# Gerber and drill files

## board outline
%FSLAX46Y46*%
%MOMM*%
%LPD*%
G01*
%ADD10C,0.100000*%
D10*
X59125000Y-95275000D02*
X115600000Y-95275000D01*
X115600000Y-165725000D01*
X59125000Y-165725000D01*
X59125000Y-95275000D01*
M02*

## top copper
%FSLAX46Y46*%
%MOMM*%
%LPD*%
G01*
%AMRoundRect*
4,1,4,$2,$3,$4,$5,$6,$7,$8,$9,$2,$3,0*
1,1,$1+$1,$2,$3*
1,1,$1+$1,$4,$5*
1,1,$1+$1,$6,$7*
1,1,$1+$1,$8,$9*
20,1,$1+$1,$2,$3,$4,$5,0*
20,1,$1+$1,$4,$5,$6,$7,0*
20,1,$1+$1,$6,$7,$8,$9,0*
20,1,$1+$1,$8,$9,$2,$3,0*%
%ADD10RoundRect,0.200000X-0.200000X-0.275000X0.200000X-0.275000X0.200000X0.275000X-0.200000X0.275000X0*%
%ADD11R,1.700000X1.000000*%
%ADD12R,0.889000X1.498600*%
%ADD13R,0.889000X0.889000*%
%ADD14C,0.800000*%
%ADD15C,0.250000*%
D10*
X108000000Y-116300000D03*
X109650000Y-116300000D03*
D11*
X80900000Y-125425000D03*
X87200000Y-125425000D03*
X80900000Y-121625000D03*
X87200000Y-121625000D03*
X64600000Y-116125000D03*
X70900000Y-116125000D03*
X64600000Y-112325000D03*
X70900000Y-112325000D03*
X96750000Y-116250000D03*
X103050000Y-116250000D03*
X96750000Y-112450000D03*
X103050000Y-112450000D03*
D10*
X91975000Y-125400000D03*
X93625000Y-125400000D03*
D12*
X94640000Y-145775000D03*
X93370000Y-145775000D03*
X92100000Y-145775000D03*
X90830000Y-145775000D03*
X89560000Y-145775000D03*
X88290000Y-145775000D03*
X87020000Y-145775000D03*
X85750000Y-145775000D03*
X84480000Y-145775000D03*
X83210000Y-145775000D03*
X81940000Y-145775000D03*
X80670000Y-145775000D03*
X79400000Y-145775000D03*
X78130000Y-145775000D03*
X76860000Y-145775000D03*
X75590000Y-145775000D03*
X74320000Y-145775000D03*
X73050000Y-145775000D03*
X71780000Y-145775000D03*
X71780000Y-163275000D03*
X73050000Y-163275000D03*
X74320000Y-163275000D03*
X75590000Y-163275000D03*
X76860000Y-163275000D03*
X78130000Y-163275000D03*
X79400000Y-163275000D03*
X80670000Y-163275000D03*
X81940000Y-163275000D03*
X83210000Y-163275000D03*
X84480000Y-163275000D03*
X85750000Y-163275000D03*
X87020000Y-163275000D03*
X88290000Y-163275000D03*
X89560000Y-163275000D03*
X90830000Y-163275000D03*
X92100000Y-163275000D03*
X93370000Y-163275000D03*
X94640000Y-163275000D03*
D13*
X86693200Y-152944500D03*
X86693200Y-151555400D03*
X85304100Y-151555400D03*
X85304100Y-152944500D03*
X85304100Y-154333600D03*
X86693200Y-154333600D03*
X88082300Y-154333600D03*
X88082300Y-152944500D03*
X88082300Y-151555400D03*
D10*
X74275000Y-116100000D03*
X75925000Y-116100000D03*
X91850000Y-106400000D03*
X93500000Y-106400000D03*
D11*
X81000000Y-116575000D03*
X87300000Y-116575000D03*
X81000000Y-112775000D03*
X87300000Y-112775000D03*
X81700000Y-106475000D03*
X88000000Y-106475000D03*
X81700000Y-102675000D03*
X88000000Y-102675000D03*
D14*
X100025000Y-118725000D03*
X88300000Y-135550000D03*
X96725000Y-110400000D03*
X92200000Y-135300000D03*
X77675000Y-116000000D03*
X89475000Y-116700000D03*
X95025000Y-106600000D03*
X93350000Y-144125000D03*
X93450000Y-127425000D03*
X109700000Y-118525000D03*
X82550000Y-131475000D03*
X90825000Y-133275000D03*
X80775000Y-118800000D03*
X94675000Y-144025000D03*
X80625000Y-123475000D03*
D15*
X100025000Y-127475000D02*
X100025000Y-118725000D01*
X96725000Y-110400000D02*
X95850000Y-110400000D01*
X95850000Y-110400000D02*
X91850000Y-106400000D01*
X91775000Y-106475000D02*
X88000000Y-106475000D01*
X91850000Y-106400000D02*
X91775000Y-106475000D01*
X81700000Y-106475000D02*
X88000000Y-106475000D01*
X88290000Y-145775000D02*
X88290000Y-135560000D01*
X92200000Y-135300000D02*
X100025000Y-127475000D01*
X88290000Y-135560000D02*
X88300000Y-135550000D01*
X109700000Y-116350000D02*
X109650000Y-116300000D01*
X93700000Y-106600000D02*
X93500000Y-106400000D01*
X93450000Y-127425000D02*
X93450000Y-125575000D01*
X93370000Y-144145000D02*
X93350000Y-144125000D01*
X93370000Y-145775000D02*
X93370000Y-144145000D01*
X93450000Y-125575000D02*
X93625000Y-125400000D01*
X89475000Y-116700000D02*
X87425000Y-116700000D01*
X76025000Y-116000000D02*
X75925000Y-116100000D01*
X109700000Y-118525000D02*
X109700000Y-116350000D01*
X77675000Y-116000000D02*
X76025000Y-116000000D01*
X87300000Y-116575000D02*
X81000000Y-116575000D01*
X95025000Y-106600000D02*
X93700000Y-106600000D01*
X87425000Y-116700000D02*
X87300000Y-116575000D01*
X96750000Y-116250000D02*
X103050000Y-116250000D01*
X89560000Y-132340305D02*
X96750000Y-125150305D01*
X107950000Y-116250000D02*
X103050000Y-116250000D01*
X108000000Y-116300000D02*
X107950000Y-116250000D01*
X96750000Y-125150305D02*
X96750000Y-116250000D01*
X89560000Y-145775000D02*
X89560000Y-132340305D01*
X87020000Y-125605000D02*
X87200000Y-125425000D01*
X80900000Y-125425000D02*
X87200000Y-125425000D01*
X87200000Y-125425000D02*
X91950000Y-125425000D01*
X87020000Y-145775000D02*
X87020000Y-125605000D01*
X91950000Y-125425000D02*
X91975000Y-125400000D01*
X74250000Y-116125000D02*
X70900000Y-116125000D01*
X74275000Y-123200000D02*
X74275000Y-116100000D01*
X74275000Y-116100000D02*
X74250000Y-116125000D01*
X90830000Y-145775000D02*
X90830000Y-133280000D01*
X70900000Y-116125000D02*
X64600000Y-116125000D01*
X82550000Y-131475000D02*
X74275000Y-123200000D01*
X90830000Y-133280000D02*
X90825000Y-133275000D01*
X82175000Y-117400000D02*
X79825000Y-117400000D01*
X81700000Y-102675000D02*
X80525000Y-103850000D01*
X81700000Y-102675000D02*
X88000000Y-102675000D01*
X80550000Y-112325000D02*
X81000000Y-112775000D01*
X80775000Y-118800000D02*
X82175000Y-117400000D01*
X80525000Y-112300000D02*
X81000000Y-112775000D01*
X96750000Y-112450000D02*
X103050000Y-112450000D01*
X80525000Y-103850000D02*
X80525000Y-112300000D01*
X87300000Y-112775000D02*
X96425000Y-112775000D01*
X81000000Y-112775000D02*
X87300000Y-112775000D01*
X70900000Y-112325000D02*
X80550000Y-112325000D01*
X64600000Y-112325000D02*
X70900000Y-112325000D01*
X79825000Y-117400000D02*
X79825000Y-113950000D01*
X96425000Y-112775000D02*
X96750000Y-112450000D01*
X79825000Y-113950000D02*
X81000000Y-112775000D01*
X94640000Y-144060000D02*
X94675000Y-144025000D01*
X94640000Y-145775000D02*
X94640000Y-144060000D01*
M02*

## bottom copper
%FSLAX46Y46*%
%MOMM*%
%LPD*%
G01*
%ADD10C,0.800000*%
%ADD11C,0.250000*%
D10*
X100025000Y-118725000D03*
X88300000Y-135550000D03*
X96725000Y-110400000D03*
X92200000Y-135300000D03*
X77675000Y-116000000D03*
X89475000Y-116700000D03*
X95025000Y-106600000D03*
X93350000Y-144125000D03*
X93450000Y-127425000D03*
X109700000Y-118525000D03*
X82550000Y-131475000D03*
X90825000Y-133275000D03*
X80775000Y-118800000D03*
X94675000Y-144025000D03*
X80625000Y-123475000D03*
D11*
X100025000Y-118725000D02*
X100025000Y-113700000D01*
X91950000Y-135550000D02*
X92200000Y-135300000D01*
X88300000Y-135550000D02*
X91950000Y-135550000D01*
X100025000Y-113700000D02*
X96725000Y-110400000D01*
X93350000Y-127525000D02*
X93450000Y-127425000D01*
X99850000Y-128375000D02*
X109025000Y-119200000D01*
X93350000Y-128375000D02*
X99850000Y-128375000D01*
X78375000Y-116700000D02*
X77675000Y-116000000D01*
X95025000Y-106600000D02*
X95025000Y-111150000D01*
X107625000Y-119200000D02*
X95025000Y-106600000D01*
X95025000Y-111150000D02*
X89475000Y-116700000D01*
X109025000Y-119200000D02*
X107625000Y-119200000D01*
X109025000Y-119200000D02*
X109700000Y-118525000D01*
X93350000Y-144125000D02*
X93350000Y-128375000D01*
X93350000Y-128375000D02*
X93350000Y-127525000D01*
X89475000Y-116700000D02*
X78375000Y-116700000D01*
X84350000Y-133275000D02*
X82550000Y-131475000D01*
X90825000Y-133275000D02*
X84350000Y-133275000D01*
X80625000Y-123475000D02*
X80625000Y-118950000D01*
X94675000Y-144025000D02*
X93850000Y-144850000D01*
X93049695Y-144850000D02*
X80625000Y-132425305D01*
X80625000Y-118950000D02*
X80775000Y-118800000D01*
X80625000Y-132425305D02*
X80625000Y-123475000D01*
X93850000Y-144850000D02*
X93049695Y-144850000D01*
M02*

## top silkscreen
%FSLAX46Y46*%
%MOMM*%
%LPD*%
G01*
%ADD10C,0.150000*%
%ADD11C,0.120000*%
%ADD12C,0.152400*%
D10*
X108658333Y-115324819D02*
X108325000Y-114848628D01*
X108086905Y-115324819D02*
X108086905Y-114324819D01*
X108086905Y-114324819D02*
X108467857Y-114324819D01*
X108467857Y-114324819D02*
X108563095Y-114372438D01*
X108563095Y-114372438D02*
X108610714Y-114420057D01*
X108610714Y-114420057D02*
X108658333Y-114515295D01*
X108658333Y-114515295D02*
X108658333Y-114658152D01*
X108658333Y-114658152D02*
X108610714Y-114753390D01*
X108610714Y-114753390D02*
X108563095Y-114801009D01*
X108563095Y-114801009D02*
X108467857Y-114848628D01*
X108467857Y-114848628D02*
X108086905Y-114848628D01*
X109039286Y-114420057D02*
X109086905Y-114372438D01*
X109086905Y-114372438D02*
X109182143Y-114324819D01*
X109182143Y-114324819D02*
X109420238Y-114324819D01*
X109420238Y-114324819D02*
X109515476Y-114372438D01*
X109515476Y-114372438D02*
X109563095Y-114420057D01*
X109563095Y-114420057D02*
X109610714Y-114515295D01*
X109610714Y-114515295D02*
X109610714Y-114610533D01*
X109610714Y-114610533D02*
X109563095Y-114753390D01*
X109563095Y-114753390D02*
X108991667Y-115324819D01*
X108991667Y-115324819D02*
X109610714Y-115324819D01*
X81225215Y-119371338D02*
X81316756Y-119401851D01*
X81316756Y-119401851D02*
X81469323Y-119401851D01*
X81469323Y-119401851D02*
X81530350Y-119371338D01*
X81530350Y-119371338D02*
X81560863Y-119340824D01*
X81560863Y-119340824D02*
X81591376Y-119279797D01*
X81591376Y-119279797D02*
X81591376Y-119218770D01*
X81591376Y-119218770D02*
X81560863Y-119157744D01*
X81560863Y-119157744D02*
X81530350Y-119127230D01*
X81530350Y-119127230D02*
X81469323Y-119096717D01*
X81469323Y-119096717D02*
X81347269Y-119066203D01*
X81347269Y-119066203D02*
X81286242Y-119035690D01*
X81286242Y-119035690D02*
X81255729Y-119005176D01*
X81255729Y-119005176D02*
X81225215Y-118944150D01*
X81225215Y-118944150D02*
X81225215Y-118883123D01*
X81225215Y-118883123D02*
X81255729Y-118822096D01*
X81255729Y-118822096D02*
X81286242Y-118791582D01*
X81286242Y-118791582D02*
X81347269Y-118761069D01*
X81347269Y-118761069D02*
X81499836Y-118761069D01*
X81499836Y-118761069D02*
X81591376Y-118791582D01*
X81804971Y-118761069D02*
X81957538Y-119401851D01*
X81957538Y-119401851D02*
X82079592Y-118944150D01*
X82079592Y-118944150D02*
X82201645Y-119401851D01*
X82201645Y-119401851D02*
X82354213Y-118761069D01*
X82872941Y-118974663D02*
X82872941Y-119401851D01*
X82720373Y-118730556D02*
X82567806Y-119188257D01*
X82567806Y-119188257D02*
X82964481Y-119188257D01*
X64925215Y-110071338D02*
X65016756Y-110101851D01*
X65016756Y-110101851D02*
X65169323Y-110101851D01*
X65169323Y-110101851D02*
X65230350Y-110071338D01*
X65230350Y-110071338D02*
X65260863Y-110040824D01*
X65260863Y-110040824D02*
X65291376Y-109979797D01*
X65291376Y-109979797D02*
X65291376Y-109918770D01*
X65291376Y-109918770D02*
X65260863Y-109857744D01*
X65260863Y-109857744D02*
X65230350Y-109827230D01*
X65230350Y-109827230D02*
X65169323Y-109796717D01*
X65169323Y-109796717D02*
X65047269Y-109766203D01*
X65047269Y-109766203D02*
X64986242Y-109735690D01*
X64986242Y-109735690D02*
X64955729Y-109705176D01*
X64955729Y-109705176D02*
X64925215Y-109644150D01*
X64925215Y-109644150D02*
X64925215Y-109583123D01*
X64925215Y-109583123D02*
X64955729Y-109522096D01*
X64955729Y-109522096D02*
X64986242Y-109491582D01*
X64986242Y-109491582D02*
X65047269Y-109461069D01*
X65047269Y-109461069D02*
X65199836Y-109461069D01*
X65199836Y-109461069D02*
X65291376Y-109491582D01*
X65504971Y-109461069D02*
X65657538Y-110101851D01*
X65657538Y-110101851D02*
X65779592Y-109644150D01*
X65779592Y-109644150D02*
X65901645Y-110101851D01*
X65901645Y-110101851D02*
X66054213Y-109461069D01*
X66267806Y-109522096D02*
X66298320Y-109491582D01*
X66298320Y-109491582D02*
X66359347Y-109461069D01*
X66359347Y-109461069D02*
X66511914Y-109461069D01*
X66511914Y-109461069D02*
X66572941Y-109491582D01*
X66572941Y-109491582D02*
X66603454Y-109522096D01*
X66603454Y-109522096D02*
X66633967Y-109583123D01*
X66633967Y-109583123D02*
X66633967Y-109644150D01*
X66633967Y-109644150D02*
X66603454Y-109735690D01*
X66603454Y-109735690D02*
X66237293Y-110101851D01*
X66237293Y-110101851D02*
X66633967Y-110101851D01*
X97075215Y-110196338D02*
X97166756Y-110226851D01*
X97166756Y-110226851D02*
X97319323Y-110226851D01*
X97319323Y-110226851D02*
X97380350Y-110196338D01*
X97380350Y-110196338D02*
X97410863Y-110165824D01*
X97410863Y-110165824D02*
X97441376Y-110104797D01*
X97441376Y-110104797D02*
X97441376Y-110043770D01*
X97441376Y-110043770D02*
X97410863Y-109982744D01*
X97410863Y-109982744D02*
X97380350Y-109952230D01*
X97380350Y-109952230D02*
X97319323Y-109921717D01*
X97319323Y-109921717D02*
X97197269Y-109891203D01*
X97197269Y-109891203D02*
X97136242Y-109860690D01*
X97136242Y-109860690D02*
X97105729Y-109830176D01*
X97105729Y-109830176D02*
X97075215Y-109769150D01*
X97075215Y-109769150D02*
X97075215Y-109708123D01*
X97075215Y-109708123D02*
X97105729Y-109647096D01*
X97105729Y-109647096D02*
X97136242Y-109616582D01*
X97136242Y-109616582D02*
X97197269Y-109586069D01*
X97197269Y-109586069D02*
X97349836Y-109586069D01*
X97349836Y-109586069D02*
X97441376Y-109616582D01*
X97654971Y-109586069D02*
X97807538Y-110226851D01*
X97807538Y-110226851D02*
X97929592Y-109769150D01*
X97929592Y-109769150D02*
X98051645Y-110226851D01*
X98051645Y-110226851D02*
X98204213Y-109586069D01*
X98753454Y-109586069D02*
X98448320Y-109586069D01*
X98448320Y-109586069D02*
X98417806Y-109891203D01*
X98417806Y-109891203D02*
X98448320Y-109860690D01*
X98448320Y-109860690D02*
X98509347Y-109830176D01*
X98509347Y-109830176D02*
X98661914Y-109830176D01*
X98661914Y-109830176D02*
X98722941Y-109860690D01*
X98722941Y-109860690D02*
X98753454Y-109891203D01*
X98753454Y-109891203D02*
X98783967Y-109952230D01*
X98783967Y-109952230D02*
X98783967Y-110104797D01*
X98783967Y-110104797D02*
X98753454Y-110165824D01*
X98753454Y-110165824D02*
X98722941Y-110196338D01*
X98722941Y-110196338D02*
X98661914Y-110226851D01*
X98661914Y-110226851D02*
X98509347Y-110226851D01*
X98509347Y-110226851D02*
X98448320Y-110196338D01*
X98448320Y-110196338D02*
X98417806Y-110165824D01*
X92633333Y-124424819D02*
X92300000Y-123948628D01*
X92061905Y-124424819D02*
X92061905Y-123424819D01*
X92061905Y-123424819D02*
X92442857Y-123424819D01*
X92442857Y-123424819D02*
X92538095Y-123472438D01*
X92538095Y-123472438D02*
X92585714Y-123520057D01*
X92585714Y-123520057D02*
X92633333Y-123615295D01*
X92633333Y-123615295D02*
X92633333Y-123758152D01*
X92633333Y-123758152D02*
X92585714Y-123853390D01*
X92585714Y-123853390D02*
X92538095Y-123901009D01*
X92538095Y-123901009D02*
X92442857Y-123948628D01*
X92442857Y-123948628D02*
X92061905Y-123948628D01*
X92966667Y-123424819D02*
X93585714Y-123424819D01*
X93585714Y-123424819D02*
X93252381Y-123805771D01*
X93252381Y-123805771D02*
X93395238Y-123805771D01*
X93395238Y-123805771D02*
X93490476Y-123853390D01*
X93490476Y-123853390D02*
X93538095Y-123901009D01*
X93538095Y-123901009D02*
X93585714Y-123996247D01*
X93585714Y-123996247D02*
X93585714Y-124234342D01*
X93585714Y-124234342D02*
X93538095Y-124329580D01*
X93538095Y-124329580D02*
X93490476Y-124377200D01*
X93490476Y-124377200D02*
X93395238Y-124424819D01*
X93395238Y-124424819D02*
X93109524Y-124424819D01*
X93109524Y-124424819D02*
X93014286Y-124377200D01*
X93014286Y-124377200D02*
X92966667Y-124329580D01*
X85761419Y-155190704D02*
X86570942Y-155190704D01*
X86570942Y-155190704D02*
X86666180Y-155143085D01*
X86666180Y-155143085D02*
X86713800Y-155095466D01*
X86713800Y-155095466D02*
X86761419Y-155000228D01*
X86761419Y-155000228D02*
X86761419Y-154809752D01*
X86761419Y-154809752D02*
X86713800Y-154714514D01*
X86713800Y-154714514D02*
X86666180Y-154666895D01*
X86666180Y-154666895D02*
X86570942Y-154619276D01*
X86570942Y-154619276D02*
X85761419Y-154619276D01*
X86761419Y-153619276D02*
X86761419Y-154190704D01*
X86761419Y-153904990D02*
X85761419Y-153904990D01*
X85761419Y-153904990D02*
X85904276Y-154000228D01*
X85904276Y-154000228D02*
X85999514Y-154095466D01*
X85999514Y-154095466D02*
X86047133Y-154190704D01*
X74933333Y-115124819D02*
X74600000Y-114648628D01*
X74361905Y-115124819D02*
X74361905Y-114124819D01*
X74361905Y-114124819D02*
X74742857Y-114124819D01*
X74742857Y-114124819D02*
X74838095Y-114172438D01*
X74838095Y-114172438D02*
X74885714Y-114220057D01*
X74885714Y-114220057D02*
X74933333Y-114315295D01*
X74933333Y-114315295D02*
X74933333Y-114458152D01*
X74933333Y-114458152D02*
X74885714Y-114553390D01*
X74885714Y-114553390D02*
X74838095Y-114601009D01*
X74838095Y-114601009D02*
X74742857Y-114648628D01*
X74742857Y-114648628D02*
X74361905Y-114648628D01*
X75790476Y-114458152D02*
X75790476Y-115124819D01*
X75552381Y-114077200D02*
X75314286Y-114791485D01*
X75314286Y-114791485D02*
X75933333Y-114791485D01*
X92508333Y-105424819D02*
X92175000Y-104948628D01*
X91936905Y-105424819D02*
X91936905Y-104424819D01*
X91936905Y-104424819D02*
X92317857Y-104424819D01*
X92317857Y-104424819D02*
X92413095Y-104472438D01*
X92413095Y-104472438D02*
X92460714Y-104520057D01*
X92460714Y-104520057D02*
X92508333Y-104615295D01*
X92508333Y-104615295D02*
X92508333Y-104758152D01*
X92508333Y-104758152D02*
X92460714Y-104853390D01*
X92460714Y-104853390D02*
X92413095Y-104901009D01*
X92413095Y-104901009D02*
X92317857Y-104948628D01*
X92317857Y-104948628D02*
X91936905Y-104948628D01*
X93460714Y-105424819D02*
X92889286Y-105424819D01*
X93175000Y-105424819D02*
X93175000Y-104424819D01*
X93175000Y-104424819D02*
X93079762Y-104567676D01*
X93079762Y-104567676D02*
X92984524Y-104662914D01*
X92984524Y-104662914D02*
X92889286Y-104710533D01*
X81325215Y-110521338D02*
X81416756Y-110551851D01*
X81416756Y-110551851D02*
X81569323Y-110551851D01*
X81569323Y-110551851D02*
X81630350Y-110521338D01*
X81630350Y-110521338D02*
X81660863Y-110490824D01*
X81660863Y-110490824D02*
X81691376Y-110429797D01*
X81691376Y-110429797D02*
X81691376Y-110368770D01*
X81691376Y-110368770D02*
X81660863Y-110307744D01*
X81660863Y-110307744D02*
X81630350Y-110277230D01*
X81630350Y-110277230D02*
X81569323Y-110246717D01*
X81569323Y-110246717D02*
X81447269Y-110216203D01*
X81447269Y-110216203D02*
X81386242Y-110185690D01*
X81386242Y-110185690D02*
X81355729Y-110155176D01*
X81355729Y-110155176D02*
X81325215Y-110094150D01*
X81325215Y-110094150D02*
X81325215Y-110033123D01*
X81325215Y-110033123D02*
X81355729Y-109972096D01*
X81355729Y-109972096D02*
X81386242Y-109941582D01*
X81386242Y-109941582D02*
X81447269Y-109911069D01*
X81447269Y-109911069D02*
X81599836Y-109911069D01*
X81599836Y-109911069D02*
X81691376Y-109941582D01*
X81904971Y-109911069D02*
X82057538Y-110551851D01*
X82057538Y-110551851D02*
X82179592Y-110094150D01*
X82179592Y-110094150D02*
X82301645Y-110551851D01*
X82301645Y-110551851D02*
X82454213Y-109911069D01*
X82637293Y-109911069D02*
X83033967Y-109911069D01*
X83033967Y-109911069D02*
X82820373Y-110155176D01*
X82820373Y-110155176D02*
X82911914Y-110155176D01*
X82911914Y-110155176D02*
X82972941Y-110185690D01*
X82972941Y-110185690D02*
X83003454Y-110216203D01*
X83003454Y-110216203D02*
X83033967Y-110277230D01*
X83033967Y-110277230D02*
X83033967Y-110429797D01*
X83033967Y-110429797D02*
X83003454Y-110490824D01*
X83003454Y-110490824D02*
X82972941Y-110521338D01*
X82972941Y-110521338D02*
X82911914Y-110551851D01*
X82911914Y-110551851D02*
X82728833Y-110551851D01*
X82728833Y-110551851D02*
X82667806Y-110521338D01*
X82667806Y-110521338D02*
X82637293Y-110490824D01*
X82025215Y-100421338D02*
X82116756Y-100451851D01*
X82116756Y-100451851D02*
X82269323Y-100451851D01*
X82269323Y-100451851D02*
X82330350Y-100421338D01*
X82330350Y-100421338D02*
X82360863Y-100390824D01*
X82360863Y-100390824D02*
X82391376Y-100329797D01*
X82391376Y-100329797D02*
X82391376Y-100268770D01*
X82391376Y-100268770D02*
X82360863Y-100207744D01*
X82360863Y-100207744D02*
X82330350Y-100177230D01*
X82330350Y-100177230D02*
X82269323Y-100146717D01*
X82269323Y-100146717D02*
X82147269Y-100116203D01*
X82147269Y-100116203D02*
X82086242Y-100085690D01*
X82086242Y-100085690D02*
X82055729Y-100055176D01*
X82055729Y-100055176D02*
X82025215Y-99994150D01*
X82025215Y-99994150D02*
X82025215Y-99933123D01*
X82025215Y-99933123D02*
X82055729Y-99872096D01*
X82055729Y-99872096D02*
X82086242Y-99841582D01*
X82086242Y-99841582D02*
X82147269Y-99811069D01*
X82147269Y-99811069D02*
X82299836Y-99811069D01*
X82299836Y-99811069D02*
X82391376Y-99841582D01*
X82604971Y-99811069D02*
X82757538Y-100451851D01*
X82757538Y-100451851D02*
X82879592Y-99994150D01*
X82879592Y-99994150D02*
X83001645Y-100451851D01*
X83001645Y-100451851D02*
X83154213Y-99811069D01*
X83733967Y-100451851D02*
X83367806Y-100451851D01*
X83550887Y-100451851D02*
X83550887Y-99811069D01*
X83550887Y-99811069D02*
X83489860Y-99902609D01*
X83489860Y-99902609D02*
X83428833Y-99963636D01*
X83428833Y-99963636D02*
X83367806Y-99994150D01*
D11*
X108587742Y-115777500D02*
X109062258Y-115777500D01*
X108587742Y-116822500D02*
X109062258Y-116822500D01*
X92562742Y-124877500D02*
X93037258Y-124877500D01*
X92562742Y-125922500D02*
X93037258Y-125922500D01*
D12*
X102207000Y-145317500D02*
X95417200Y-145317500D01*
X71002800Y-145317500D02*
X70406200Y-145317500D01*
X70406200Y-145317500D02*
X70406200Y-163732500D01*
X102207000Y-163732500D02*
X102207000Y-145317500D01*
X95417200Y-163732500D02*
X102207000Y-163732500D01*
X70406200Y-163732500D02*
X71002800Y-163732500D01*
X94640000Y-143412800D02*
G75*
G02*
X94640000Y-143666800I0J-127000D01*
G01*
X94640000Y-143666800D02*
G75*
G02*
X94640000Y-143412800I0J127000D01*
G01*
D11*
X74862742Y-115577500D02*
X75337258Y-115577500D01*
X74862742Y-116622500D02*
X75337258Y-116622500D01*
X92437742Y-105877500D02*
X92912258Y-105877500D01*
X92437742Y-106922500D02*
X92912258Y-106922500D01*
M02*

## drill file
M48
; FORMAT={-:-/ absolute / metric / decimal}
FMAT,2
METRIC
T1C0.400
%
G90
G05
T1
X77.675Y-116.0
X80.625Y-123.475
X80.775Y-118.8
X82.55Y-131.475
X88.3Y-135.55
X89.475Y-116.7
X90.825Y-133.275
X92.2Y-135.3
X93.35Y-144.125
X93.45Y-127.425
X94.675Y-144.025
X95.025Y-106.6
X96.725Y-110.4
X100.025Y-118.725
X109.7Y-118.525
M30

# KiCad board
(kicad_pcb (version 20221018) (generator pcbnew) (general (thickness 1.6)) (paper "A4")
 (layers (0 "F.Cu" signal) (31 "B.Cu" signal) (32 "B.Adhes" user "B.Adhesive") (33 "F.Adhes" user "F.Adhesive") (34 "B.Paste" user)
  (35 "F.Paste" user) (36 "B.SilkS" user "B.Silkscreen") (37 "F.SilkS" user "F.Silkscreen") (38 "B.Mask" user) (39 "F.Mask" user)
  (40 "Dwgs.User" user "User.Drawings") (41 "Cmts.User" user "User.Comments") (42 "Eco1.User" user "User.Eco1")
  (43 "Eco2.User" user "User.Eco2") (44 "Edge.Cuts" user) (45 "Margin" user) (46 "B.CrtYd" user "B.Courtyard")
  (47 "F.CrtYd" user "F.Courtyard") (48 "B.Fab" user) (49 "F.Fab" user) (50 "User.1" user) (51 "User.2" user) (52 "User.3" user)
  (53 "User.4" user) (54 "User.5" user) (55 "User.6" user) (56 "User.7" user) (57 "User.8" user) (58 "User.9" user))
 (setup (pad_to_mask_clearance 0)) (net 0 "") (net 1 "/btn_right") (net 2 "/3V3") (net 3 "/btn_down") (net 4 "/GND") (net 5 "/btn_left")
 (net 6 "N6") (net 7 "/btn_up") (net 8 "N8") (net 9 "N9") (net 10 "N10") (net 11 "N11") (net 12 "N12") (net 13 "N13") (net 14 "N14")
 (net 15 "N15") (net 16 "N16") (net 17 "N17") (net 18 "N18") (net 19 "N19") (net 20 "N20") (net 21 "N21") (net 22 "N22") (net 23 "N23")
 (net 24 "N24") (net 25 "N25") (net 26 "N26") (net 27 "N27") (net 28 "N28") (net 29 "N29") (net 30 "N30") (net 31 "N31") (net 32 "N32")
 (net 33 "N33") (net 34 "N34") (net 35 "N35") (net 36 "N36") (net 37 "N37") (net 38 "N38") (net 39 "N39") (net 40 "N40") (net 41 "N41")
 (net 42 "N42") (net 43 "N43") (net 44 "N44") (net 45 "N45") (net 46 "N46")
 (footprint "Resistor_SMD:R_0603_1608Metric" (layer "F.Cu") (at 108.825 116.3)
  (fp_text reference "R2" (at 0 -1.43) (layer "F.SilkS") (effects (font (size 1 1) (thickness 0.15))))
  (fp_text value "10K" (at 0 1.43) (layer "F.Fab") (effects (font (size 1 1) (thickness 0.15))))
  (fp_line (start -0.237258 -0.5225) (end 0.237258 -0.5225) (stroke (width 0.12) (type solid)) (layer "F.SilkS"))
  (fp_line (start -0.237258 0.5225) (end 0.237258 0.5225) (stroke (width 0.12) (type solid)) (layer "F.SilkS"))
  (pad "1" smd roundrect (at -0.825 0) (size 0.8 0.95) (layers "F.Cu" "F.Paste" "F.Mask") (roundrect_rratio 0.25) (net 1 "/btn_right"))
  (pad "2" smd roundrect (at 0.825 0) (size 0.8 0.95) (layers "F.Cu" "F.Paste" "F.Mask") (roundrect_rratio 0.25) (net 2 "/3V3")))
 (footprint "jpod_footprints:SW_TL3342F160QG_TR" (layer "F.Cu") (at 84.05 123.525)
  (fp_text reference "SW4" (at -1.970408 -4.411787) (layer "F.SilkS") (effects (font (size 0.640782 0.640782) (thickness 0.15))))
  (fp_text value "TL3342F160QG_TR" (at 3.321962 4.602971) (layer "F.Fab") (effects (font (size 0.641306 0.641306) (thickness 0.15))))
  (pad "1" smd rect (at -3.15 1.9) (size 1.7 1) (layers "F.Cu" "F.Paste" "F.Mask") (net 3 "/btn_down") (solder_mask_margin 0.102))
  (pad "2" smd rect (at 3.15 1.9) (size 1.7 1) (layers "F.Cu" "F.Paste" "F.Mask") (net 3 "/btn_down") (solder_mask_margin 0.102))
  (pad "3" smd rect (at -3.15 -1.9) (size 1.7 1) (layers "F.Cu" "F.Paste" "F.Mask") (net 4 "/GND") (solder_mask_margin 0.102))
  (pad "4" smd rect (at 3.15 -1.9) (size 1.7 1) (layers "F.Cu" "F.Paste" "F.Mask") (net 4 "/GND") (solder_mask_margin 0.102)))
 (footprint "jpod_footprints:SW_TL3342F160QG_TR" (layer "F.Cu") (at 67.75 114.225)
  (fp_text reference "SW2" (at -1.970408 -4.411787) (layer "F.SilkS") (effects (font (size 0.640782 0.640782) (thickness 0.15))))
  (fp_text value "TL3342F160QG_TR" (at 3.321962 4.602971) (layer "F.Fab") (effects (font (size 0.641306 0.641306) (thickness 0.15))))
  (pad "1" smd rect (at -3.15 1.9) (size 1.7 1) (layers "F.Cu" "F.Paste" "F.Mask") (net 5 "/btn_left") (solder_mask_margin 0.102))
  (pad "2" smd rect (at 3.15 1.9) (size 1.7 1) (layers "F.Cu" "F.Paste" "F.Mask") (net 5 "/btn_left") (solder_mask_margin 0.102))
  (pad "3" smd rect (at -3.15 -1.9) (size 1.7 1) (layers "F.Cu" "F.Paste" "F.Mask") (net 4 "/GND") (solder_mask_margin 0.102))
  (pad "4" smd rect (at 3.15 -1.9) (size 1.7 1) (layers "F.Cu" "F.Paste" "F.Mask") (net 4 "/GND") (solder_mask_margin 0.102)))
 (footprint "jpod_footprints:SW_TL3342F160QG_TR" (layer "F.Cu") (at 99.9 114.35)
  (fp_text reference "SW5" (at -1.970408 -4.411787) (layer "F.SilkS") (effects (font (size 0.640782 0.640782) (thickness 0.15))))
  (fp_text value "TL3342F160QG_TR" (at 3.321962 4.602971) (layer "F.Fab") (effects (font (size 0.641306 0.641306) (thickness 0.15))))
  (pad "1" smd rect (at -3.15 1.9) (size 1.7 1) (layers "F.Cu" "F.Paste" "F.Mask") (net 1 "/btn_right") (solder_mask_margin 0.102))
  (pad "2" smd rect (at 3.15 1.9) (size 1.7 1) (layers "F.Cu" "F.Paste" "F.Mask") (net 1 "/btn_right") (solder_mask_margin 0.102))
  (pad "3" smd rect (at -3.15 -1.9) (size 1.7 1) (layers "F.Cu" "F.Paste" "F.Mask") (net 4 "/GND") (solder_mask_margin 0.102))
  (pad "4" smd rect (at 3.15 -1.9) (size 1.7 1) (layers "F.Cu" "F.Paste" "F.Mask") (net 4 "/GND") (solder_mask_margin 0.102)))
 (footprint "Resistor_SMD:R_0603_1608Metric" (layer "F.Cu") (at 92.8 125.4)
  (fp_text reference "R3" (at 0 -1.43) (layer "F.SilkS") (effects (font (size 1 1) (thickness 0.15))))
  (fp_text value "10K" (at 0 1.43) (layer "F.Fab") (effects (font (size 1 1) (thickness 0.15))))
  (fp_line (start -0.237258 -0.5225) (end 0.237258 -0.5225) (stroke (width 0.12) (type solid)) (layer "F.SilkS"))
  (fp_line (start -0.237258 0.5225) (end 0.237258 0.5225) (stroke (width 0.12) (type solid)) (layer "F.SilkS"))
  (pad "1" smd roundrect (at -0.825 0) (size 0.8 0.95) (layers "F.Cu" "F.Paste" "F.Mask") (roundrect_rratio 0.25) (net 3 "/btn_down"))
  (pad "2" smd roundrect (at 0.825 0) (size 0.8 0.95) (layers "F.Cu" "F.Paste" "F.Mask") (roundrect_rratio 0.25) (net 2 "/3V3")))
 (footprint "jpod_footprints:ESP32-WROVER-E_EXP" (layer "F.Cu") (at 86.3066 154.525 -90)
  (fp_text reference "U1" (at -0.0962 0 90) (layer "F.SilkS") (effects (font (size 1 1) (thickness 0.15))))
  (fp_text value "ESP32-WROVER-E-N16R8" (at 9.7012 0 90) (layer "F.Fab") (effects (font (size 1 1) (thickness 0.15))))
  (fp_line (start -9.2075 -15.9004) (end -9.2075 -9.1106) (stroke (width 0.1524) (type solid)) (layer "F.SilkS"))
  (fp_line (start -9.2075 15.3038) (end -9.2075 15.9004) (stroke (width 0.1524) (type solid)) (layer "F.SilkS"))
  (fp_line (start -9.2075 15.9004) (end 9.2075 15.9004) (stroke (width 0.1524) (type solid)) (layer "F.SilkS"))
  (fp_line (start 9.2075 -15.9004) (end -9.2075 -15.9004) (stroke (width 0.1524) (type solid)) (layer "F.SilkS"))
  (fp_line (start 9.2075 -9.1106) (end 9.2075 -15.9004) (stroke (width 0.1524) (type solid)) (layer "F.SilkS"))
  (fp_line (start 9.2075 15.9004) (end 9.2075 15.3038) (stroke (width 0.1524) (type solid)) (layer "F.SilkS"))
  (fp_arc (start -11.1122 -8.3334) (mid -10.9852 -8.4604) (end -10.8582 -8.3334) (stroke (width 0.1524) (type solid)) (layer "F.SilkS"))
  (fp_arc (start -10.8582 -8.3334) (mid -10.9852 -8.2064) (end -11.1122 -8.3334) (stroke (width 0.1524) (type solid)) (layer "F.SilkS"))
  (pad "1" smd rect (at -8.75 -8.3334 270) (size 1.4986 0.889) (layers "F.Cu" "F.Paste" "F.Mask") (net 4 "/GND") (solder_mask_margin 0.102))
  (pad "2" smd rect (at -8.75 -7.0634 270) (size 1.4986 0.889) (layers "F.Cu" "F.Paste" "F.Mask") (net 2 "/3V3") (solder_mask_margin 0.102))
  (pad "3" smd rect (at -8.75 -5.7934 270) (size 1.4986 0.889) (layers "F.Cu" "F.Paste" "F.Mask") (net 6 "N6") (solder_mask_margin 0.102))
  (pad "4" smd rect (at -8.75 -4.5234 270) (size 1.4986 0.889) (layers "F.Cu" "F.Paste" "F.Mask") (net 5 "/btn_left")
   (solder_mask_margin 0.102))
  (pad "5" smd rect (at -8.75 -3.2534 270) (size 1.4986 0.889) (layers "F.Cu" "F.Paste" "F.Mask") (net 1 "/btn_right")
   (solder_mask_margin 0.102))
  (pad "6" smd rect (at -8.75 -1.9834 270) (size 1.4986 0.889) (layers "F.Cu" "F.Paste" "F.Mask") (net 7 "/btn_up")
   (solder_mask_margin 0.102))
  (pad "7" smd rect (at -8.75 -0.7134 270) (size 1.4986 0.889) (layers "F.Cu" "F.Paste" "F.Mask") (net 3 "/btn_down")
   (solder_mask_margin 0.102))
  (pad "8" smd rect (at -8.75 0.5566 270) (size 1.4986 0.889) (layers "F.Cu" "F.Paste" "F.Mask") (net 2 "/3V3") (solder_mask_margin 0.102))
  (pad "9" smd rect (at -8.75 1.8266 270) (size 1.4986 0.889) (layers "F.Cu" "F.Paste" "F.Mask") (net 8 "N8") (solder_mask_margin 0.102))
  (pad "10" smd rect (at -8.75 3.0966 270) (size 1.4986 0.889) (layers "F.Cu" "F.Paste" "F.Mask") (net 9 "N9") (solder_mask_margin 0.102))
  (pad "11" smd rect (at -8.75 4.3666 270) (size 1.4986 0.889) (layers "F.Cu" "F.Paste" "F.Mask") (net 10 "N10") (solder_mask_margin 0.102))
  (pad "12" smd rect (at -8.75 5.6366 270) (size 1.4986 0.889) (layers "F.Cu" "F.Paste" "F.Mask") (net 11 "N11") (solder_mask_margin 0.102))
  (pad "13" smd rect (at -8.75 6.9066 270) (size 1.4986 0.889) (layers "F.Cu" "F.Paste" "F.Mask") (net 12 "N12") (solder_mask_margin 0.102))
  (pad "14" smd rect (at -8.75 8.1766 270) (size 1.4986 0.889) (layers "F.Cu" "F.Paste" "F.Mask") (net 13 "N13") (solder_mask_margin 0.102))
  (pad "15" smd rect (at -8.75 9.4466 270) (size 1.4986 0.889) (layers "F.Cu" "F.Paste" "F.Mask") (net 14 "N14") (solder_mask_margin 0.102))
  (pad "16" smd rect (at -8.75 10.7166 270) (size 1.4986 0.889) (layers "F.Cu" "F.Paste" "F.Mask") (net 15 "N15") (solder_mask_margin 0.102))
  (pad "17" smd rect (at -8.75 11.9866 270) (size 1.4986 0.889) (layers "F.Cu" "F.Paste" "F.Mask") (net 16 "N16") (solder_mask_margin 0.102))
  (pad "18" smd rect (at -8.75 13.2566 270) (size 1.4986 0.889) (layers "F.Cu" "F.Paste" "F.Mask") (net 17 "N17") (solder_mask_margin 0.102))
  (pad "19" smd rect (at -8.75 14.5266 270) (size 1.4986 0.889) (layers "F.Cu" "F.Paste" "F.Mask") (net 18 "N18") (solder_mask_margin 0.102))
  (pad "20" smd rect (at 8.75 14.5266 270) (size 1.4986 0.889) (layers "F.Cu" "F.Paste" "F.Mask") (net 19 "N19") (solder_mask_margin 0.102))
  (pad "21" smd rect (at 8.75 13.2566 270) (size 1.4986 0.889) (layers "F.Cu" "F.Paste" "F.Mask") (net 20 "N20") (solder_mask_margin 0.102))
  (pad "22" smd rect (at 8.75 11.9866 270) (size 1.4986 0.889) (layers "F.Cu" "F.Paste" "F.Mask") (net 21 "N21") (solder_mask_margin 0.102))
  (pad "23" smd rect (at 8.75 10.7166 270) (size 1.4986 0.889) (layers "F.Cu" "F.Paste" "F.Mask") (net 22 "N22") (solder_mask_margin 0.102))
  (pad "24" smd rect (at 8.75 9.4466 270) (size 1.4986 0.889) (layers "F.Cu" "F.Paste" "F.Mask") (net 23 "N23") (solder_mask_margin 0.102))
  (pad "25" smd rect (at 8.75 8.1766 270) (size 1.4986 0.889) (layers "F.Cu" "F.Paste" "F.Mask") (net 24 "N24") (solder_mask_margin 0.102))
  (pad "26" smd rect (at 8.75 6.9066 270) (size 1.4986 0.889) (layers "F.Cu" "F.Paste" "F.Mask") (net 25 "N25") (solder_mask_margin 0.102))
  (pad "27" smd rect (at 8.75 5.6366 270) (size 1.4986 0.889) (layers "F.Cu" "F.Paste" "F.Mask") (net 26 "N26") (solder_mask_margin 0.102))
  (pad "28" smd rect (at 8.75 4.3666 270) (size 1.4986 0.889) (layers "F.Cu" "F.Paste" "F.Mask") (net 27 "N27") (solder_mask_margin 0.102))
  (pad "29" smd rect (at 8.75 3.0966 270) (size 1.4986 0.889) (layers "F.Cu" "F.Paste" "F.Mask") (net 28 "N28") (solder_mask_margin 0.102))
  (pad "30" smd rect (at 8.75 1.8266 270) (size 1.4986 0.889) (layers "F.Cu" "F.Paste" "F.Mask") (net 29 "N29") (solder_mask_margin 0.102))
  (pad "31" smd rect (at 8.75 0.5566 270) (size 1.4986 0.889) (layers "F.Cu" "F.Paste" "F.Mask") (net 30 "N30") (solder_mask_margin 0.102))
  (pad "32" smd rect (at 8.75 -0.7134 270) (size 1.4986 0.889) (layers "F.Cu" "F.Paste" "F.Mask") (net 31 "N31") (solder_mask_margin 0.102))
  (pad "33" smd rect (at 8.75 -1.9834 270) (size 1.4986 0.889) (layers "F.Cu" "F.Paste" "F.Mask") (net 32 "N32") (solder_mask_margin 0.102))
  (pad "34" smd rect (at 8.75 -3.2534 270) (size 1.4986 0.889) (layers "F.Cu" "F.Paste" "F.Mask") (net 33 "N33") (solder_mask_margin 0.102))
  (pad "35" smd rect (at 8.75 -4.5234 270) (size 1.4986 0.889) (layers "F.Cu" "F.Paste" "F.Mask") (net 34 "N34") (solder_mask_margin 0.102))
  (pad "36" smd rect (at 8.75 -5.7934 270) (size 1.4986 0.889) (layers "F.Cu" "F.Paste" "F.Mask") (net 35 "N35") (solder_mask_margin 0.102))
  (pad "37" smd rect (at 8.75 -7.0634 270) (size 1.4986 0.889) (layers "F.Cu" "F.Paste" "F.Mask") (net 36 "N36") (solder_mask_margin 0.102))
  (pad "38" smd rect (at 8.75 -8.3334 270) (size 1.4986 0.889) (layers "F.Cu" "F.Paste" "F.Mask") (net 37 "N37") (solder_mask_margin 0.102))
  (pad "39" smd rect (at -1.5805 -0.3866 270) (size 0.889 0.889) (layers "F.Cu" "F.Paste" "F.Mask") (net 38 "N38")
   (solder_mask_margin 0.102))
  (pad "40" smd rect (at -2.9696 -0.3866 270) (size 0.889 0.889) (layers "F.Cu" "F.Paste" "F.Mask") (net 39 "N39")
   (solder_mask_margin 0.102))
  (pad "41" smd rect (at -2.9696 1.0025 270) (size 0.889 0.889) (layers "F.Cu" "F.Paste" "F.Mask") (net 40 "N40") (solder_mask_margin 0.102))
  (pad "42" smd rect (at -1.5805 1.0025 270) (size 0.889 0.889) (layers "F.Cu" "F.Paste" "F.Mask") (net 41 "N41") (solder_mask_margin 0.102))
  (pad "43" smd rect (at -0.1914 1.0025 270) (size 0.889 0.889) (layers "F.Cu" "F.Paste" "F.Mask") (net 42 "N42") (solder_mask_margin 0.102))
  (pad "44" smd rect (at -0.1914 -0.3866 270) (size 0.889 0.889) (layers "F.Cu" "F.Paste" "F.Mask") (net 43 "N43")
   (solder_mask_margin 0.102))
  (pad "45" smd rect (at -0.1914 -1.7757 270) (size 0.889 0.889) (layers "F.Cu" "F.Paste" "F.Mask") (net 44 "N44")
   (solder_mask_margin 0.102))
  (pad "46" smd rect (at -1.5805 -1.7757 270) (size 0.889 0.889) (layers "F.Cu" "F.Paste" "F.Mask") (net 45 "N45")
   (solder_mask_margin 0.102))
  (pad "47" smd rect (at -2.9696 -1.7757 270) (size 0.889 0.889) (layers "F.Cu" "F.Paste" "F.Mask") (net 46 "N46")
   (solder_mask_margin 0.102)))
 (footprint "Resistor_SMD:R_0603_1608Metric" (layer "F.Cu") (at 75.1 116.1)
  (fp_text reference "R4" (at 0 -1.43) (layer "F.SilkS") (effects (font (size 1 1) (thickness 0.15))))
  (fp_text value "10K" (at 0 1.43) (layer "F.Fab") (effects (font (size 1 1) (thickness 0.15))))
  (fp_line (start -0.237258 -0.5225) (end 0.237258 -0.5225) (stroke (width 0.12) (type solid)) (layer "F.SilkS"))
  (fp_line (start -0.237258 0.5225) (end 0.237258 0.5225) (stroke (width 0.12) (type solid)) (layer "F.SilkS"))
  (pad "1" smd roundrect (at -0.825 0) (size 0.8 0.95) (layers "F.Cu" "F.Paste" "F.Mask") (roundrect_rratio 0.25) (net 5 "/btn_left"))
  (pad "2" smd roundrect (at 0.825 0) (size 0.8 0.95) (layers "F.Cu" "F.Paste" "F.Mask") (roundrect_rratio 0.25) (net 2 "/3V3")))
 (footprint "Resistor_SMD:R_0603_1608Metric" (layer "F.Cu") (at 92.675 106.4)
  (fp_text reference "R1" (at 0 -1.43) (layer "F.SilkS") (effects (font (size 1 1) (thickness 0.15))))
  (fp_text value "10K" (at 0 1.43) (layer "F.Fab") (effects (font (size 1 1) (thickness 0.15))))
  (fp_line (start -0.237258 -0.5225) (end 0.237258 -0.5225) (stroke (width 0.12) (type solid)) (layer "F.SilkS"))
  (fp_line (start -0.237258 0.5225) (end 0.237258 0.5225) (stroke (width 0.12) (type solid)) (layer "F.SilkS"))
  (pad "1" smd roundrect (at -0.825 0) (size 0.8 0.95) (layers "F.Cu" "F.Paste" "F.Mask") (roundrect_rratio 0.25) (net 7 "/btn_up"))
  (pad "2" smd roundrect (at 0.825 0) (size 0.8 0.95) (layers "F.Cu" "F.Paste" "F.Mask") (roundrect_rratio 0.25) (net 2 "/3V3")))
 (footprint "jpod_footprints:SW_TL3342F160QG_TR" (layer "F.Cu") (at 84.15 114.675)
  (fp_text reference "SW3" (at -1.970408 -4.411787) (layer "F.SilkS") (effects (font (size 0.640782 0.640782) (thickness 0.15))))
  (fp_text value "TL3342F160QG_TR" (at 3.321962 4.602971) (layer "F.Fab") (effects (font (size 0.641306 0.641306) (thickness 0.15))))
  (pad "1" smd rect (at -3.15 1.9) (size 1.7 1) (layers "F.Cu" "F.Paste" "F.Mask") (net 2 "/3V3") (solder_mask_margin 0.102))
  (pad "2" smd rect (at 3.15 1.9) (size 1.7 1) (layers "F.Cu" "F.Paste" "F.Mask") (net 2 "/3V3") (solder_mask_margin 0.102))
  (pad "3" smd rect (at -3.15 -1.9) (size 1.7 1) (layers "F.Cu" "F.Paste" "F.Mask") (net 4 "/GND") (solder_mask_margin 0.102))
  (pad "4" smd rect (at 3.15 -1.9) (size 1.7 1) (layers "F.Cu" "F.Paste" "F.Mask") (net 4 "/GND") (solder_mask_margin 0.102)))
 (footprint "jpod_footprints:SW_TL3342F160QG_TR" (layer "F.Cu") (at 84.85 104.575)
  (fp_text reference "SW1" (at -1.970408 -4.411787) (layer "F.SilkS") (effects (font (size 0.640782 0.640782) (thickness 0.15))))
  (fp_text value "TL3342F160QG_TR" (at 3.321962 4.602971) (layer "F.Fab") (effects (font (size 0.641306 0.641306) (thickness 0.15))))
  (pad "1" smd rect (at -3.15 1.9) (size 1.7 1) (layers "F.Cu" "F.Paste" "F.Mask") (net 7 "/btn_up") (solder_mask_margin 0.102))
  (pad "2" smd rect (at 3.15 1.9) (size 1.7 1) (layers "F.Cu" "F.Paste" "F.Mask") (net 7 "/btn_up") (solder_mask_margin 0.102))
  (pad "3" smd rect (at -3.15 -1.9) (size 1.7 1) (layers "F.Cu" "F.Paste" "F.Mask") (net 4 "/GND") (solder_mask_margin 0.102))
  (pad "4" smd rect (at 3.15 -1.9) (size 1.7 1) (layers "F.Cu" "F.Paste" "F.Mask") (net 4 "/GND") (solder_mask_margin 0.102)))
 (gr_rect (start 59.125 95.275) (end 115.6 165.725) (stroke (width 0.1) (type default)) (fill none) (layer "Edge.Cuts"))
 (segment (start 100.025 127.475) (end 100.025 118.725) (width 0.25) (layer "F.Cu") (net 7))
 (segment (start 96.725 110.4) (end 95.85 110.4) (width 0.25) (layer "F.Cu") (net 7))
 (segment (start 95.85 110.4) (end 91.85 106.4) (width 0.25) (layer "F.Cu") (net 7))
 (segment (start 91.775 106.475) (end 88 106.475) (width 0.25) (layer "F.Cu") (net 7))
 (segment (start 91.85 106.4) (end 91.775 106.475) (width 0.25) (layer "F.Cu") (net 7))
 (segment (start 81.7 106.475) (end 88 106.475) (width 0.25) (layer "F.Cu") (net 7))
 (segment (start 88.29 145.775) (end 88.29 135.56) (width 0.25) (layer "F.Cu") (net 7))
 (segment (start 92.2 135.3) (end 100.025 127.475) (width 0.25) (layer "F.Cu") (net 7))
 (segment (start 88.29 135.56) (end 88.3 135.55) (width 0.25) (layer "F.Cu") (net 7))
 (via (at 100.025 118.725) (size 0.8) (drill 0.4) (layers "F.Cu" "B.Cu") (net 7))
 (via (at 88.3 135.55) (size 0.8) (drill 0.4) (layers "F.Cu" "B.Cu") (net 7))
 (via (at 96.725 110.4) (size 0.8) (drill 0.4) (layers "F.Cu" "B.Cu") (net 7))
 (via (at 92.2 135.3) (size 0.8) (drill 0.4) (layers "F.Cu" "B.Cu") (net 7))
 (segment (start 100.025 118.725) (end 100.025 113.7) (width 0.25) (layer "B.Cu") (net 7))
 (segment (start 91.95 135.55) (end 92.2 135.3) (width 0.25) (layer "B.Cu") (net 7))
 (segment (start 88.3 135.55) (end 91.95 135.55) (width 0.25) (layer "B.Cu") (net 7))
 (segment (start 100.025 113.7) (end 96.725 110.4) (width 0.25) (layer "B.Cu") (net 7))
 (segment (start 109.7 116.35) (end 109.65 116.3) (width 0.25) (layer "F.Cu") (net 2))
 (segment (start 93.7 106.6) (end 93.5 106.4) (width 0.25) (layer "F.Cu") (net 2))
 (segment (start 93.45 127.425) (end 93.45 125.575) (width 0.25) (layer "F.Cu") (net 2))
 (segment (start 93.37 144.145) (end 93.35 144.125) (width 0.25) (layer "F.Cu") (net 2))
 (segment (start 93.37 145.775) (end 93.37 144.145) (width 0.25) (layer "F.Cu") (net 2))
 (segment (start 93.45 125.575) (end 93.625 125.4) (width 0.25) (layer "F.Cu") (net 2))
 (segment (start 89.475 116.7) (end 87.425 116.7) (width 0.25) (layer "F.Cu") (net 2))
 (segment (start 76.025 116) (end 75.925 116.1) (width 0.25) (layer "F.Cu") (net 2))
 (segment (start 109.7 118.525) (end 109.7 116.35) (width 0.25) (layer "F.Cu") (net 2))
 (segment (start 77.675 116) (end 76.025 116) (width 0.25) (layer "F.Cu") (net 2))
 (segment (start 87.3 116.575) (end 81 116.575) (width 0.25) (layer "F.Cu") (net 2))
 (segment (start 95.025 106.6) (end 93.7 106.6) (width 0.25) (layer "F.Cu") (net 2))
 (segment (start 87.425 116.7) (end 87.3 116.575) (width 0.25) (layer "F.Cu") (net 2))
 (via (at 77.675 116) (size 0.8) (drill 0.4) (layers "F.Cu" "B.Cu") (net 2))
 (via (at 89.475 116.7) (size 0.8) (drill 0.4) (layers "F.Cu" "B.Cu") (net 2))
 (via (at 95.025 106.6) (size 0.8) (drill 0.4) (layers "F.Cu" "B.Cu") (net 2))
 (via (at 93.35 144.125) (size 0.8) (drill 0.4) (layers "F.Cu" "B.Cu") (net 2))
 (via (at 93.45 127.425) (size 0.8) (drill 0.4) (layers "F.Cu" "B.Cu") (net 2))
 (via (at 109.7 118.525) (size 0.8) (drill 0.4) (layers "F.Cu" "B.Cu") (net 2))
 (segment (start 93.35 127.525) (end 93.45 127.425) (width 0.25) (layer "B.Cu") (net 2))
 (segment (start 99.85 128.375) (end 109.025 119.2) (width 0.25) (layer "B.Cu") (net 2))
 (segment (start 93.35 128.375) (end 99.85 128.375) (width 0.25) (layer "B.Cu") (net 2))
 (segment (start 78.375 116.7) (end 77.675 116) (width 0.25) (layer "B.Cu") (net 2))
 (segment (start 95.025 106.6) (end 95.025 111.15) (width 0.25) (layer "B.Cu") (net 2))
 (segment (start 107.625 119.2) (end 95.025 106.6) (width 0.25) (layer "B.Cu") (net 2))
 (segment (start 95.025 111.15) (end 89.475 116.7) (width 0.25) (layer "B.Cu") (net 2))
 (segment (start 109.025 119.2) (end 107.625 119.2) (width 0.25) (layer "B.Cu") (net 2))
 (segment (start 109.025 119.2) (end 109.7 118.525) (width 0.25) (layer "B.Cu") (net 2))
 (segment (start 93.35 144.125) (end 93.35 128.375) (width 0.25) (layer "B.Cu") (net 2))
 (segment (start 93.35 128.375) (end 93.35 127.525) (width 0.25) (layer "B.Cu") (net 2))
 (segment (start 89.475 116.7) (end 78.375 116.7) (width 0.25) (layer "B.Cu") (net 2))
 (segment (start 96.75 116.25) (end 103.05 116.25) (width 0.25) (layer "F.Cu") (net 1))
 (segment (start 89.56 132.340305) (end 96.75 125.150305) (width 0.25) (layer "F.Cu") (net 1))
 (segment (start 107.95 116.25) (end 103.05 116.25) (width 0.25) (layer "F.Cu") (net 1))
 (segment (start 108 116.3) (end 107.95 116.25) (width 0.25) (layer "F.Cu") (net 1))
 (segment (start 96.75 125.150305) (end 96.75 116.25) (width 0.25) (layer "F.Cu") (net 1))
 (segment (start 89.56 145.775) (end 89.56 132.340305) (width 0.25) (layer "F.Cu") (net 1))
 (segment (start 87.02 125.605) (end 87.2 125.425) (width 0.25) (layer "F.Cu") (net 3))
 (segment (start 80.9 125.425) (end 87.2 125.425) (width 0.25) (layer "F.Cu") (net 3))
 (segment (start 87.2 125.425) (end 91.95 125.425) (width 0.25) (layer "F.Cu") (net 3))
 (segment (start 87.02 145.775) (end 87.02 125.605) (width 0.25) (layer "F.Cu") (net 3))
 (segment (start 91.95 125.425) (end 91.975 125.4) (width 0.25) (layer "F.Cu") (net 3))
 (segment (start 74.25 116.125) (end 70.9 116.125) (width 0.25) (layer "F.Cu") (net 5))
 (segment (start 74.275 123.2) (end 74.275 116.1) (width 0.25) (layer "F.Cu") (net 5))
 (segment (start 74.275 116.1) (end 74.25 116.125) (width 0.25) (layer "F.Cu") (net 5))
 (segment (start 90.83 145.775) (end 90.83 133.28) (width 0.25) (layer "F.Cu") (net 5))
 (segment (start 70.9 116.125) (end 64.6 116.125) (width 0.25) (layer "F.Cu") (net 5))
 (segment (start 82.55 131.475) (end 74.275 123.2) (width 0.25) (layer "F.Cu") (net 5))
 (segment (start 90.83 133.28) (end 90.825 133.275) (width 0.25) (layer "F.Cu") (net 5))
 (via (at 82.55 131.475) (size 0.8) (drill 0.4) (layers "F.Cu" "B.Cu") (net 5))
 (via (at 90.825 133.275) (size 0.8) (drill 0.4) (layers "F.Cu" "B.Cu") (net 5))
 (segment (start 84.35 133.275) (end 82.55 131.475) (width 0.25) (layer "B.Cu") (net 5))
 (segment (start 90.825 133.275) (end 84.35 133.275) (width 0.25) (layer "B.Cu") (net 5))
 (segment (start 82.175 117.4) (end 79.825 117.4) (width 0.25) (layer "F.Cu") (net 4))
 (segment (start 81.7 102.675) (end 80.525 103.85) (width 0.25) (layer "F.Cu") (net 4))
 (segment (start 81.7 102.675) (end 88 102.675) (width 0.25) (layer "F.Cu") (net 4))
 (segment (start 80.55 112.325) (end 81 112.775) (width 0.25) (layer "F.Cu") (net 4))
 (segment (start 80.775 118.8) (end 82.175 117.4) (width 0.25) (layer "F.Cu") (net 4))
 (segment (start 80.525 112.3) (end 81 112.775) (width 0.25) (layer "F.Cu") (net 4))
 (segment (start 96.75 112.45) (end 103.05 112.45) (width 0.25) (layer "F.Cu") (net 4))
 (segment (start 80.525 103.85) (end 80.525 112.3) (width 0.25) (layer "F.Cu") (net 4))
 (segment (start 87.3 112.775) (end 96.425 112.775) (width 0.25) (layer "F.Cu") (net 4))
 (segment (start 81 112.775) (end 87.3 112.775) (width 0.25) (layer "F.Cu") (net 4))
 (segment (start 70.9 112.325) (end 80.55 112.325) (width 0.25) (layer "F.Cu") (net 4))
 (segment (start 64.6 112.325) (end 70.9 112.325) (width 0.25) (layer "F.Cu") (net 4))
 (segment (start 79.825 117.4) (end 79.825 113.95) (width 0.25) (layer "F.Cu") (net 4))
 (segment (start 96.425 112.775) (end 96.75 112.45) (width 0.25) (layer "F.Cu") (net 4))
 (segment (start 79.825 113.95) (end 81 112.775) (width 0.25) (layer "F.Cu") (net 4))
 (segment (start 94.64 144.06) (end 94.675 144.025) (width 0.25) (layer "F.Cu") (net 4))
 (segment (start 94.64 145.775) (end 94.64 144.06) (width 0.25) (layer "F.Cu") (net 4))
 (via (at 80.775 118.8) (size 0.8) (drill 0.4) (layers "F.Cu" "B.Cu") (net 4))
 (via (at 94.675 144.025) (size 0.8) (drill 0.4) (layers "F.Cu" "B.Cu") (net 4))
 (via (at 80.625 123.475) (size 0.8) (drill 0.4) (layers "F.Cu" "B.Cu") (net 4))
 (segment (start 80.625 123.475) (end 80.625 118.95) (width 0.25) (layer "B.Cu") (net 4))
 (segment (start 94.675 144.025) (end 93.85 144.85) (width 0.25) (layer "B.Cu") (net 4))
 (segment (start 93.049695 144.85) (end 80.625 132.425305) (width 0.25) (layer "B.Cu") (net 4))
 (segment (start 80.625 118.95) (end 80.775 118.8) (width 0.25) (layer "B.Cu") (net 4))
 (segment (start 80.625 132.425305) (end 80.625 123.475) (width 0.25) (layer "B.Cu") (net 4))
 (segment (start 93.85 144.85) (end 93.049695 144.85) (width 0.25) (layer "B.Cu") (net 4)))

